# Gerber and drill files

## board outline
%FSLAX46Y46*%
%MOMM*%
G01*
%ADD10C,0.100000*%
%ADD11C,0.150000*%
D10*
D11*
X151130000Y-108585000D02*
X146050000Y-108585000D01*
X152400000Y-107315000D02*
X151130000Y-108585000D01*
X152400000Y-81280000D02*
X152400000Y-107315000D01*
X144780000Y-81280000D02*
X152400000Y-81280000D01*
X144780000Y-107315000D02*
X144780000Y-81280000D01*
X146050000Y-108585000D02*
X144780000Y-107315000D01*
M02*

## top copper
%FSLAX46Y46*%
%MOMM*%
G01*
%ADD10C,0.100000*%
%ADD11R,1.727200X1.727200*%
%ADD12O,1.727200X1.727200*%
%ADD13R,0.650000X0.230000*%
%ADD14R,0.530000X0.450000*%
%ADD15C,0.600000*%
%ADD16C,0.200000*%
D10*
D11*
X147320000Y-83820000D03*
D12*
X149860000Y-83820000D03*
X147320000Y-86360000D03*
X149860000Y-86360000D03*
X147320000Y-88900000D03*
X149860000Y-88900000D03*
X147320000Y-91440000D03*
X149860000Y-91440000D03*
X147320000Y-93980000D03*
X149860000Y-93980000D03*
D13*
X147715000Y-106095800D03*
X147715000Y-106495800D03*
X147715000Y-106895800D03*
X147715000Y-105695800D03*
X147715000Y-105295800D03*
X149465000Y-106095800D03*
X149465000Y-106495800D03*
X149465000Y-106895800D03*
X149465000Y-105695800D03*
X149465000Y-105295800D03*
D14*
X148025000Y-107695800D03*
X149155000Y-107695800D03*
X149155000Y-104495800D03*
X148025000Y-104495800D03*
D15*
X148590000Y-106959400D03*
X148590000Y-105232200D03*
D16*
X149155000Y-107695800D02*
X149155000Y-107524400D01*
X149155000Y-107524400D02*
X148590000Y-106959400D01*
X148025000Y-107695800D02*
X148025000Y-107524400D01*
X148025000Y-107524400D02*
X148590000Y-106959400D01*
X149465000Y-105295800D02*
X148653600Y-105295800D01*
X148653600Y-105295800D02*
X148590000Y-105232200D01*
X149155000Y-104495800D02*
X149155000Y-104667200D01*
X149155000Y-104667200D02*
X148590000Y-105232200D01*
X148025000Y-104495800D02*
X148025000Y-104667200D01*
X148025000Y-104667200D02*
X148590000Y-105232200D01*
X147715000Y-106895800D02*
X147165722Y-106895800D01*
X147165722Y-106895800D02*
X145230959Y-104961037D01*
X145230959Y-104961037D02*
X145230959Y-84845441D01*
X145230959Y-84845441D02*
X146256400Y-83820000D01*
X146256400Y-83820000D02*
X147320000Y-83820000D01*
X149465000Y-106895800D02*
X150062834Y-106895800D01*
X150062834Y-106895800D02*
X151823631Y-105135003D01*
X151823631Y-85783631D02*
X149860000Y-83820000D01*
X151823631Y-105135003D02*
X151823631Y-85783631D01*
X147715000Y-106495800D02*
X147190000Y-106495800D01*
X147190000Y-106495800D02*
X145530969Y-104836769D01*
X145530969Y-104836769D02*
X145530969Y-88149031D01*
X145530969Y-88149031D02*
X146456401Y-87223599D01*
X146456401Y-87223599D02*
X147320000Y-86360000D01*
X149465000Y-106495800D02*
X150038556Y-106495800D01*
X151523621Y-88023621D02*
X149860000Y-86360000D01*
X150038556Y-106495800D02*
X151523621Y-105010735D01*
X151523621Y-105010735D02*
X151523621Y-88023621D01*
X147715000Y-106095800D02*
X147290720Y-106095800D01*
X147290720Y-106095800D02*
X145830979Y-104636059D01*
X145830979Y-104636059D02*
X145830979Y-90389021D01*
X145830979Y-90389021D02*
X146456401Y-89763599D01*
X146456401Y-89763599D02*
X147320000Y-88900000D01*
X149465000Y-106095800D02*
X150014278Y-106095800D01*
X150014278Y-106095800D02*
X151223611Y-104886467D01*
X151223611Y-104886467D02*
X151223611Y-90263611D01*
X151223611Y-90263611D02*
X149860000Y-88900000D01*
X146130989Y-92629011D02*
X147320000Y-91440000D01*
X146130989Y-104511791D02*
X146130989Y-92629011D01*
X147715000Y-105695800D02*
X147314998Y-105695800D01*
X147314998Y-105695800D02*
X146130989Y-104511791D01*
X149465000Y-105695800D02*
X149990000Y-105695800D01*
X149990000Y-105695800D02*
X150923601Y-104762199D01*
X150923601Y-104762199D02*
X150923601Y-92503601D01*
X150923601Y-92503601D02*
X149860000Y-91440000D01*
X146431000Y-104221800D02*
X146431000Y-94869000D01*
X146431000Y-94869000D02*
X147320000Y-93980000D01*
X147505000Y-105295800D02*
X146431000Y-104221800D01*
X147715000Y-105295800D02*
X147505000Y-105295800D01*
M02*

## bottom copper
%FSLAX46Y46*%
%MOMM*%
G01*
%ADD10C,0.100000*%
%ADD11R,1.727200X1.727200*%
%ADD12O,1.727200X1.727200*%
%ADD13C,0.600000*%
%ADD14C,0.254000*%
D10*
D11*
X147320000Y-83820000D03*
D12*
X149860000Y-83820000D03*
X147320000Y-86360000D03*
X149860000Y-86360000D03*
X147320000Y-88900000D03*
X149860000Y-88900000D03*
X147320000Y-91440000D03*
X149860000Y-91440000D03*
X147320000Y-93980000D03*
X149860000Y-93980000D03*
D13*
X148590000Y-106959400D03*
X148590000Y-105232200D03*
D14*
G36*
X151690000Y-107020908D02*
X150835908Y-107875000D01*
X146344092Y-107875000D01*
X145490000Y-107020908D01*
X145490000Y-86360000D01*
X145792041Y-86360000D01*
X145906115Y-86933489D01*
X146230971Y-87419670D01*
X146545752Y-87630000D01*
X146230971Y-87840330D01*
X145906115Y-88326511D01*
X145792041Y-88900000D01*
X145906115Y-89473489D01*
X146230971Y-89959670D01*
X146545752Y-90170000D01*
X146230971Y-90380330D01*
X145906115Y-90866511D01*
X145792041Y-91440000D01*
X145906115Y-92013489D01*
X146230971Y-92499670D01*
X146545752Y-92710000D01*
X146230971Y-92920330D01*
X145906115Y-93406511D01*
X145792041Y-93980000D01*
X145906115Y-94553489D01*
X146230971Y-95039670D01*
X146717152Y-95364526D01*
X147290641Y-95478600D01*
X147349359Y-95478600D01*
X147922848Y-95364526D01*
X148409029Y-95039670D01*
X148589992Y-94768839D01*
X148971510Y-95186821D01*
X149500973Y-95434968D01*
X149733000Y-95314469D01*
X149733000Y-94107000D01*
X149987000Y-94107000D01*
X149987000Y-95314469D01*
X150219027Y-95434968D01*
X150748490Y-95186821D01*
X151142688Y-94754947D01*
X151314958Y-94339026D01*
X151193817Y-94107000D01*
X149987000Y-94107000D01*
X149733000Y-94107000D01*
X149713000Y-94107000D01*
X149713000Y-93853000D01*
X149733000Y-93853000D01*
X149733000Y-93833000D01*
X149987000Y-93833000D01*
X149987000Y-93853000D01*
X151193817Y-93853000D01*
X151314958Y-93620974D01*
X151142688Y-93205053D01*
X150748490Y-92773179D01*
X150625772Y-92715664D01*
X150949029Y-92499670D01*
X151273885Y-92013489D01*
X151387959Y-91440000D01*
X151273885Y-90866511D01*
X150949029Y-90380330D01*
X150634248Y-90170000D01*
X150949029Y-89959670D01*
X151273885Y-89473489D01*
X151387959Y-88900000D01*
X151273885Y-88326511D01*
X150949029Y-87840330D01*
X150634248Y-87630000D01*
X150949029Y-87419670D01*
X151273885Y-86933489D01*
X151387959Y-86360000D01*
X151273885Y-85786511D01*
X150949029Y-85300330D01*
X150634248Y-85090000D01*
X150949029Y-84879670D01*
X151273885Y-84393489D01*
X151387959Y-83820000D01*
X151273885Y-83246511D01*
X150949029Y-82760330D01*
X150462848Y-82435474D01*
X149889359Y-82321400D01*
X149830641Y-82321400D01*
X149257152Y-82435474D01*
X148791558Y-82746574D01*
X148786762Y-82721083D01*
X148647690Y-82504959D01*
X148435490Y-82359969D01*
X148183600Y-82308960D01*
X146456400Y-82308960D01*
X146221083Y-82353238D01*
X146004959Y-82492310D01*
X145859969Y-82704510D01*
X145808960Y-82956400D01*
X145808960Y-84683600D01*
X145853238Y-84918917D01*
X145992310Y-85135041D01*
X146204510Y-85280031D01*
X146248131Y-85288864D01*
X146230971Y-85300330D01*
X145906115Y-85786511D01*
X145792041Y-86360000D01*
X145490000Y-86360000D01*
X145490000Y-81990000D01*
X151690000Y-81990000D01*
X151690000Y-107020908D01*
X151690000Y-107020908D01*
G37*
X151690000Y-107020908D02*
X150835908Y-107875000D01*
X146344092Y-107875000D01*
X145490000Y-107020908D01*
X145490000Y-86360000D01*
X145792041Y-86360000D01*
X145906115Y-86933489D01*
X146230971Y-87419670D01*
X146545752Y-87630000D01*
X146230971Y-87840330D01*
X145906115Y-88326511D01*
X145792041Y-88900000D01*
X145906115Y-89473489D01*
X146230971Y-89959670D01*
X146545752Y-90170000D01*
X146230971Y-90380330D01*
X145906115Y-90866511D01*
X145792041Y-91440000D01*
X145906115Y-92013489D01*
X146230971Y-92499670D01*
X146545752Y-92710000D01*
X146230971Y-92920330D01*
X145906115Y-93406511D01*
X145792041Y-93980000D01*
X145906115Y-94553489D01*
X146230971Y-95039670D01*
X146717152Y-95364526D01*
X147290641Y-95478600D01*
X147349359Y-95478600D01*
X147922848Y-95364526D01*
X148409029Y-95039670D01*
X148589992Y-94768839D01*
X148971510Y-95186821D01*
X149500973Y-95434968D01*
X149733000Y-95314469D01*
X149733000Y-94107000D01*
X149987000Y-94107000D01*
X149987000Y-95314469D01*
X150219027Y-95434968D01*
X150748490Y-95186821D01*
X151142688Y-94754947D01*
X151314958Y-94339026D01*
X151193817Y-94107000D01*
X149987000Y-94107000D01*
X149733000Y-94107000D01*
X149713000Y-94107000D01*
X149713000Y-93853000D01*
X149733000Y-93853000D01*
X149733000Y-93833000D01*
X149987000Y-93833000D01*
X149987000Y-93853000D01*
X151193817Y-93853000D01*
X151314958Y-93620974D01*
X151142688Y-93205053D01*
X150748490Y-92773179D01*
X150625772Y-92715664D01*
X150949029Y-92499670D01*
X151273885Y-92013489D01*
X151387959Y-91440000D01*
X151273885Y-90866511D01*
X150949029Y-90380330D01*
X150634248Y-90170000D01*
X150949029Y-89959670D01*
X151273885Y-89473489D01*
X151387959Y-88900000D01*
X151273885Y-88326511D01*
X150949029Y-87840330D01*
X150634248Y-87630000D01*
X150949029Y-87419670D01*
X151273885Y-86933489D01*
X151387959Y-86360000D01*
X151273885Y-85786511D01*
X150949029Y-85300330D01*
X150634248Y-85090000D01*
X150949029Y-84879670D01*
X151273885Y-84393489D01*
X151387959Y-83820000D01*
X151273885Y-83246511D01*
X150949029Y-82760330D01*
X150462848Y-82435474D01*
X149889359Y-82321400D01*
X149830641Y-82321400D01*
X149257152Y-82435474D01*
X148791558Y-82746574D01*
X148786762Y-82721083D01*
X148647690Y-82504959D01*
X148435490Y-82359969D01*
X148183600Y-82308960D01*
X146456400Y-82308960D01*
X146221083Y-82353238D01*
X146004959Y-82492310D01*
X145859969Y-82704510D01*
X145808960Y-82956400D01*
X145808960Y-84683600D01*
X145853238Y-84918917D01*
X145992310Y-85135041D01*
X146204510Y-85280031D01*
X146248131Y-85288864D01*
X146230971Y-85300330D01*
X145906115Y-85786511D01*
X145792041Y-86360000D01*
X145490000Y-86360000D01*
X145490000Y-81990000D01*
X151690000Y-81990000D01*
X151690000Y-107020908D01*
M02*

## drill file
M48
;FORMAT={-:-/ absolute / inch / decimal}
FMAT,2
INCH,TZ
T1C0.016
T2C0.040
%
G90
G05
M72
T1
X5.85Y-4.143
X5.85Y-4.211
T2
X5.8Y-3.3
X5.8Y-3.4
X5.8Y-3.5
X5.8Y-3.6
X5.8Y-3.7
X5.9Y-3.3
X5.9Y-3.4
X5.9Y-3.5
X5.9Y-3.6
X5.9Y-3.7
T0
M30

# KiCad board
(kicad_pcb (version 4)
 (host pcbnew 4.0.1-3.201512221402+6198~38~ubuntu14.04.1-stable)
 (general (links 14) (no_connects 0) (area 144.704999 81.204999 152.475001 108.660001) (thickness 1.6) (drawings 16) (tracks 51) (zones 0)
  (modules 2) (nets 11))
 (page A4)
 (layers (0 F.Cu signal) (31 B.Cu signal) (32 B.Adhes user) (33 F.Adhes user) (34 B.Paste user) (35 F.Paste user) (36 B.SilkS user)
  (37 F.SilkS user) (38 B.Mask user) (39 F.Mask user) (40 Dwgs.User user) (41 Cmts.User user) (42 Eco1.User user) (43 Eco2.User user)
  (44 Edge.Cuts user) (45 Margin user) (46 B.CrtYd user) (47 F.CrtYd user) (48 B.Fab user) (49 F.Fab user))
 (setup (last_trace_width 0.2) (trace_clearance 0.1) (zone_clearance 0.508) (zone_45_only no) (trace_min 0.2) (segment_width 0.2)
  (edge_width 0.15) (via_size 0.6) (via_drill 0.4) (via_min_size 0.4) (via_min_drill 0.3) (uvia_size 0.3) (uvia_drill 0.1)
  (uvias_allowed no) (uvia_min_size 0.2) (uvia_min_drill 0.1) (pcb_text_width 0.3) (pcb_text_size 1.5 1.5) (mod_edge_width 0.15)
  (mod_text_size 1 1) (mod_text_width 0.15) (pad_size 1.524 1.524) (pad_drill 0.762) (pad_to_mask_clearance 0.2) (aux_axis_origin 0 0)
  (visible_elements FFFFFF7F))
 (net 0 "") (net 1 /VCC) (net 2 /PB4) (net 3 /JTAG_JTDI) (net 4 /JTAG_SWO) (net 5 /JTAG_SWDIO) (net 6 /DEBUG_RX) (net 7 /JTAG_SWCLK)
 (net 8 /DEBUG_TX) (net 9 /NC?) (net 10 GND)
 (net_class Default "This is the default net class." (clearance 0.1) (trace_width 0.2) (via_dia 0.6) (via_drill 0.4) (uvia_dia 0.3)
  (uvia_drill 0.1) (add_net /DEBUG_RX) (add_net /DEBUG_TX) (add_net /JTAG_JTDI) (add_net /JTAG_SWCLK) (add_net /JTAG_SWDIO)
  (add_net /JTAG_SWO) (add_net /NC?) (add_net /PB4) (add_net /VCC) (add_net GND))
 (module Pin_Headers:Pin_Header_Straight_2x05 (layer F.Cu) (at 147.32 83.82)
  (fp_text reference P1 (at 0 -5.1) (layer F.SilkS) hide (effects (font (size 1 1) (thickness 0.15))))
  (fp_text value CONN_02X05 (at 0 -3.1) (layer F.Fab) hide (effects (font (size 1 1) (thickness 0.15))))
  (pad 1 thru_hole rect (at 0 0) (size 1.7272 1.7272) (drill 1.016) (layers *.Cu *.Mask F.SilkS) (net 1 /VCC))
  (pad 2 thru_hole oval (at 2.54 0) (size 1.7272 1.7272) (drill 1.016) (layers *.Cu *.Mask F.SilkS) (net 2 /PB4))
  (pad 3 thru_hole oval (at 0 2.54) (size 1.7272 1.7272) (drill 1.016) (layers *.Cu *.Mask F.SilkS) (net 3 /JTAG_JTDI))
  (pad 4 thru_hole oval (at 2.54 2.54) (size 1.7272 1.7272) (drill 1.016) (layers *.Cu *.Mask F.SilkS) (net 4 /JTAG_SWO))
  (pad 5 thru_hole oval (at 0 5.08) (size 1.7272 1.7272) (drill 1.016) (layers *.Cu *.Mask F.SilkS) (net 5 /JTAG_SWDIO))
  (pad 6 thru_hole oval (at 2.54 5.08) (size 1.7272 1.7272) (drill 1.016) (layers *.Cu *.Mask F.SilkS) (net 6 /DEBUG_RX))
  (pad 7 thru_hole oval (at 0 7.62) (size 1.7272 1.7272) (drill 1.016) (layers *.Cu *.Mask F.SilkS) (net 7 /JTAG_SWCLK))
  (pad 8 thru_hole oval (at 2.54 7.62) (size 1.7272 1.7272) (drill 1.016) (layers *.Cu *.Mask F.SilkS) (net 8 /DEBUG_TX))
  (pad 9 thru_hole oval (at 0 10.16) (size 1.7272 1.7272) (drill 1.016) (layers *.Cu *.Mask F.SilkS) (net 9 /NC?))
  (pad 10 thru_hole oval (at 2.54 10.16) (size 1.7272 1.7272) (drill 1.016) (layers *.Cu *.Mask F.SilkS) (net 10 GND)))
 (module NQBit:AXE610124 (layer F.Cu) (at 148.59 106.0958 180)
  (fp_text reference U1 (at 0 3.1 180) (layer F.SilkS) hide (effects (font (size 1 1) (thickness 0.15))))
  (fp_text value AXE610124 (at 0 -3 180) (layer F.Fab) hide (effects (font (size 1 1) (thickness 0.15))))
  (pad 5 smd rect (at 0.875 0 180) (size 0.65 0.23) (layers F.Cu F.Paste F.Mask) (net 5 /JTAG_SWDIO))
  (pad 3 smd rect (at 0.875 -0.4 180) (size 0.65 0.23) (layers F.Cu F.Paste F.Mask) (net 3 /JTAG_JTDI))
  (pad 1 smd rect (at 0.875 -0.8 180) (size 0.65 0.23) (layers F.Cu F.Paste F.Mask) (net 1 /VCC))
  (pad 7 smd rect (at 0.875 0.4 180) (size 0.65 0.23) (layers F.Cu F.Paste F.Mask) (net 7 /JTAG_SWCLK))
  (pad 9 smd rect (at 0.875 0.8 180) (size 0.65 0.23) (layers F.Cu F.Paste F.Mask) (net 9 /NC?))
  (pad 6 smd rect (at -0.875 0 180) (size 0.65 0.23) (layers F.Cu F.Paste F.Mask) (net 6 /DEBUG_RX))
  (pad 4 smd rect (at -0.875 -0.4 180) (size 0.65 0.23) (layers F.Cu F.Paste F.Mask) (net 4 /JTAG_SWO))
  (pad 2 smd rect (at -0.875 -0.8 180) (size 0.65 0.23) (layers F.Cu F.Paste F.Mask) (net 2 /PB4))
  (pad 8 smd rect (at -0.875 0.4 180) (size 0.65 0.23) (layers F.Cu F.Paste F.Mask) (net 8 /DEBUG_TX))
  (pad 10 smd rect (at -0.875 0.8 180) (size 0.65 0.23) (layers F.Cu F.Paste F.Mask) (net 10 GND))
  (pad P4 smd rect (at 0.565 -1.6 180) (size 0.53 0.45) (layers F.Cu F.Paste F.Mask) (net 10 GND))
  (pad P1 smd rect (at -0.565 -1.6 180) (size 0.53 0.45) (layers F.Cu F.Paste F.Mask) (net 10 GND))
  (pad P2 smd rect (at -0.565 1.6 180) (size 0.53 0.45) (layers F.Cu F.Paste F.Mask) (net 10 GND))
  (pad P3 smd rect (at 0.565 1.6 180) (size 0.53 0.45) (layers F.Cu F.Paste F.Mask) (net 10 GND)))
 (gr_line (start 151.13 108.585) (end 146.05 108.585) (layer Edge.Cuts) (width 0.15))
 (gr_line (start 152.4 107.315) (end 151.13 108.585) (layer Edge.Cuts) (width 0.15))
 (gr_line (start 152.4 81.28) (end 152.4 107.315) (layer Edge.Cuts) (width 0.15))
 (gr_line (start 144.78 81.28) (end 152.4 81.28) (layer Edge.Cuts) (width 0.15))
 (gr_line (start 144.78 107.315) (end 144.78 81.28) (layer Edge.Cuts) (width 0.15))
 (gr_line (start 146.05 108.585) (end 144.78 107.315) (layer Edge.Cuts) (width 0.15))
 (segment (start 149.155 107.6958) (end 149.155 107.5244) (width 0.2) (layer F.Cu) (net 10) (status 30))
 (segment (start 149.155 107.5244) (end 148.59 106.9594) (width 0.2) (layer F.Cu) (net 10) (status 10))
 (segment (start 148.025 107.6958) (end 148.025 107.5244) (width 0.2) (layer F.Cu) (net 10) (status 30))
 (segment (start 148.025 107.5244) (end 148.59 106.9594) (width 0.2) (layer F.Cu) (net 10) (status 10))
 (via (at 148.59 106.9594) (size 0.6) (drill 0.4) (layers F.Cu B.Cu) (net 10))
 (segment (start 149.465 105.2958) (end 148.6536 105.2958) (width 0.2) (layer F.Cu) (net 10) (status 10))
 (segment (start 148.6536 105.2958) (end 148.59 105.2322) (width 0.2) (layer F.Cu) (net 10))
 (segment (start 149.155 104.4958) (end 149.155 104.6672) (width 0.2) (layer F.Cu) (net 10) (status 30))
 (segment (start 149.155 104.6672) (end 148.59 105.2322) (width 0.2) (layer F.Cu) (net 10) (status 10))
 (segment (start 148.025 104.4958) (end 148.025 104.6672) (width 0.2) (layer F.Cu) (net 10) (status 30))
 (segment (start 148.025 104.6672) (end 148.59 105.2322) (width 0.2) (layer F.Cu) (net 10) (status 10))
 (via (at 148.59 105.2322) (size 0.6) (drill 0.4) (layers F.Cu B.Cu) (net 10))
 (segment (start 147.715 106.8958) (end 147.165722 106.8958) (width 0.2) (layer F.Cu) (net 1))
 (segment (start 147.165722 106.8958) (end 145.230959 104.961037) (width 0.2) (layer F.Cu) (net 1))
 (segment (start 145.230959 104.961037) (end 145.230959 84.845441) (width 0.2) (layer F.Cu) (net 1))
 (segment (start 145.230959 84.845441) (end 146.2564 83.82) (width 0.2) (layer F.Cu) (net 1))
 (segment (start 146.2564 83.82) (end 147.32 83.82) (width 0.2) (layer F.Cu) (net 1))
 (segment (start 149.465 106.8958) (end 150.062834 106.8958) (width 0.2) (layer F.Cu) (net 2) (status 10))
 (segment (start 150.062834 106.8958) (end 151.823631 105.135003) (width 0.2) (layer F.Cu) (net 2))
 (segment (start 151.823631 85.783631) (end 149.86 83.82) (width 0.2) (layer F.Cu) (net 2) (status 20))
 (segment (start 151.823631 105.135003) (end 151.823631 85.783631) (width 0.2) (layer F.Cu) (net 2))
 (segment (start 147.715 106.4958) (end 147.19 106.4958) (width 0.2) (layer F.Cu) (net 3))
 (segment (start 147.19 106.4958) (end 145.530969 104.836769) (width 0.2) (layer F.Cu) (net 3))
 (segment (start 145.530969 104.836769) (end 145.530969 88.149031) (width 0.2) (layer F.Cu) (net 3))
 (segment (start 145.530969 88.149031) (end 146.456401 87.223599) (width 0.2) (layer F.Cu) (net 3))
 (segment (start 146.456401 87.223599) (end 147.32 86.36) (width 0.2) (layer F.Cu) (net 3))
 (segment (start 149.465 106.4958) (end 150.038556 106.4958) (width 0.2) (layer F.Cu) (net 4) (status 10))
 (segment (start 151.523621 88.023621) (end 149.86 86.36) (width 0.2) (layer F.Cu) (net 4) (status 20))
 (segment (start 150.038556 106.4958) (end 151.523621 105.010735) (width 0.2) (layer F.Cu) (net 4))
 (segment (start 151.523621 105.010735) (end 151.523621 88.023621) (width 0.2) (layer F.Cu) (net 4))
 (segment (start 147.715 106.0958) (end 147.29072 106.0958) (width 0.2) (layer F.Cu) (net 5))
 (segment (start 147.29072 106.0958) (end 145.830979 104.636059) (width 0.2) (layer F.Cu) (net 5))
 (segment (start 145.830979 104.636059) (end 145.830979 90.389021) (width 0.2) (layer F.Cu) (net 5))
 (segment (start 145.830979 90.389021) (end 146.456401 89.763599) (width 0.2) (layer F.Cu) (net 5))
 (segment (start 146.456401 89.763599) (end 147.32 88.9) (width 0.2) (layer F.Cu) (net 5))
 (segment (start 149.465 106.0958) (end 150.014278 106.0958) (width 0.2) (layer F.Cu) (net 6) (status 10))
 (segment (start 150.014278 106.0958) (end 151.223611 104.886467) (width 0.2) (layer F.Cu) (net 6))
 (segment (start 151.223611 104.886467) (end 151.223611 90.263611) (width 0.2) (layer F.Cu) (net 6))
 (segment (start 151.223611 90.263611) (end 149.86 88.9) (width 0.2) (layer F.Cu) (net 6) (status 20))
 (segment (start 146.130989 92.629011) (end 147.32 91.44) (width 0.2) (layer F.Cu) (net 7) (status 20))
 (segment (start 146.130989 104.511791) (end 146.130989 92.629011) (width 0.2) (layer F.Cu) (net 7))
 (segment (start 147.715 105.6958) (end 147.314998 105.6958) (width 0.2) (layer F.Cu) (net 7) (status 10))
 (segment (start 147.314998 105.6958) (end 146.130989 104.511791) (width 0.2) (layer F.Cu) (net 7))
 (segment (start 149.465 105.6958) (end 149.99 105.6958) (width 0.2) (layer F.Cu) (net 8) (status 10))
 (segment (start 149.99 105.6958) (end 150.923601 104.762199) (width 0.2) (layer F.Cu) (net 8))
 (segment (start 150.923601 104.762199) (end 150.923601 92.503601) (width 0.2) (layer F.Cu) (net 8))
 (segment (start 150.923601 92.503601) (end 149.86 91.44) (width 0.2) (layer F.Cu) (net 8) (status 20))
 (segment (start 146.431 104.2218) (end 146.431 94.869) (width 0.2) (layer F.Cu) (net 9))
 (segment (start 146.431 94.869) (end 147.32 93.98) (width 0.2) (layer F.Cu) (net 9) (status 20))
 (segment (start 147.505 105.2958) (end 146.431 104.2218) (width 0.2) (layer F.Cu) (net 9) (status 10))
 (segment (start 147.715 105.2958) (end 147.505 105.2958) (width 0.2) (layer F.Cu) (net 9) (status 30))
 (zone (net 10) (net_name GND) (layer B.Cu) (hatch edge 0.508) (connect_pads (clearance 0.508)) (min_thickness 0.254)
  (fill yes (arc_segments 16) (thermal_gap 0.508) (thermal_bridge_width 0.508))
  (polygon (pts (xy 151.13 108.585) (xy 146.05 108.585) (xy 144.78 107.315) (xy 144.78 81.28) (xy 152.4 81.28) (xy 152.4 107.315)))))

